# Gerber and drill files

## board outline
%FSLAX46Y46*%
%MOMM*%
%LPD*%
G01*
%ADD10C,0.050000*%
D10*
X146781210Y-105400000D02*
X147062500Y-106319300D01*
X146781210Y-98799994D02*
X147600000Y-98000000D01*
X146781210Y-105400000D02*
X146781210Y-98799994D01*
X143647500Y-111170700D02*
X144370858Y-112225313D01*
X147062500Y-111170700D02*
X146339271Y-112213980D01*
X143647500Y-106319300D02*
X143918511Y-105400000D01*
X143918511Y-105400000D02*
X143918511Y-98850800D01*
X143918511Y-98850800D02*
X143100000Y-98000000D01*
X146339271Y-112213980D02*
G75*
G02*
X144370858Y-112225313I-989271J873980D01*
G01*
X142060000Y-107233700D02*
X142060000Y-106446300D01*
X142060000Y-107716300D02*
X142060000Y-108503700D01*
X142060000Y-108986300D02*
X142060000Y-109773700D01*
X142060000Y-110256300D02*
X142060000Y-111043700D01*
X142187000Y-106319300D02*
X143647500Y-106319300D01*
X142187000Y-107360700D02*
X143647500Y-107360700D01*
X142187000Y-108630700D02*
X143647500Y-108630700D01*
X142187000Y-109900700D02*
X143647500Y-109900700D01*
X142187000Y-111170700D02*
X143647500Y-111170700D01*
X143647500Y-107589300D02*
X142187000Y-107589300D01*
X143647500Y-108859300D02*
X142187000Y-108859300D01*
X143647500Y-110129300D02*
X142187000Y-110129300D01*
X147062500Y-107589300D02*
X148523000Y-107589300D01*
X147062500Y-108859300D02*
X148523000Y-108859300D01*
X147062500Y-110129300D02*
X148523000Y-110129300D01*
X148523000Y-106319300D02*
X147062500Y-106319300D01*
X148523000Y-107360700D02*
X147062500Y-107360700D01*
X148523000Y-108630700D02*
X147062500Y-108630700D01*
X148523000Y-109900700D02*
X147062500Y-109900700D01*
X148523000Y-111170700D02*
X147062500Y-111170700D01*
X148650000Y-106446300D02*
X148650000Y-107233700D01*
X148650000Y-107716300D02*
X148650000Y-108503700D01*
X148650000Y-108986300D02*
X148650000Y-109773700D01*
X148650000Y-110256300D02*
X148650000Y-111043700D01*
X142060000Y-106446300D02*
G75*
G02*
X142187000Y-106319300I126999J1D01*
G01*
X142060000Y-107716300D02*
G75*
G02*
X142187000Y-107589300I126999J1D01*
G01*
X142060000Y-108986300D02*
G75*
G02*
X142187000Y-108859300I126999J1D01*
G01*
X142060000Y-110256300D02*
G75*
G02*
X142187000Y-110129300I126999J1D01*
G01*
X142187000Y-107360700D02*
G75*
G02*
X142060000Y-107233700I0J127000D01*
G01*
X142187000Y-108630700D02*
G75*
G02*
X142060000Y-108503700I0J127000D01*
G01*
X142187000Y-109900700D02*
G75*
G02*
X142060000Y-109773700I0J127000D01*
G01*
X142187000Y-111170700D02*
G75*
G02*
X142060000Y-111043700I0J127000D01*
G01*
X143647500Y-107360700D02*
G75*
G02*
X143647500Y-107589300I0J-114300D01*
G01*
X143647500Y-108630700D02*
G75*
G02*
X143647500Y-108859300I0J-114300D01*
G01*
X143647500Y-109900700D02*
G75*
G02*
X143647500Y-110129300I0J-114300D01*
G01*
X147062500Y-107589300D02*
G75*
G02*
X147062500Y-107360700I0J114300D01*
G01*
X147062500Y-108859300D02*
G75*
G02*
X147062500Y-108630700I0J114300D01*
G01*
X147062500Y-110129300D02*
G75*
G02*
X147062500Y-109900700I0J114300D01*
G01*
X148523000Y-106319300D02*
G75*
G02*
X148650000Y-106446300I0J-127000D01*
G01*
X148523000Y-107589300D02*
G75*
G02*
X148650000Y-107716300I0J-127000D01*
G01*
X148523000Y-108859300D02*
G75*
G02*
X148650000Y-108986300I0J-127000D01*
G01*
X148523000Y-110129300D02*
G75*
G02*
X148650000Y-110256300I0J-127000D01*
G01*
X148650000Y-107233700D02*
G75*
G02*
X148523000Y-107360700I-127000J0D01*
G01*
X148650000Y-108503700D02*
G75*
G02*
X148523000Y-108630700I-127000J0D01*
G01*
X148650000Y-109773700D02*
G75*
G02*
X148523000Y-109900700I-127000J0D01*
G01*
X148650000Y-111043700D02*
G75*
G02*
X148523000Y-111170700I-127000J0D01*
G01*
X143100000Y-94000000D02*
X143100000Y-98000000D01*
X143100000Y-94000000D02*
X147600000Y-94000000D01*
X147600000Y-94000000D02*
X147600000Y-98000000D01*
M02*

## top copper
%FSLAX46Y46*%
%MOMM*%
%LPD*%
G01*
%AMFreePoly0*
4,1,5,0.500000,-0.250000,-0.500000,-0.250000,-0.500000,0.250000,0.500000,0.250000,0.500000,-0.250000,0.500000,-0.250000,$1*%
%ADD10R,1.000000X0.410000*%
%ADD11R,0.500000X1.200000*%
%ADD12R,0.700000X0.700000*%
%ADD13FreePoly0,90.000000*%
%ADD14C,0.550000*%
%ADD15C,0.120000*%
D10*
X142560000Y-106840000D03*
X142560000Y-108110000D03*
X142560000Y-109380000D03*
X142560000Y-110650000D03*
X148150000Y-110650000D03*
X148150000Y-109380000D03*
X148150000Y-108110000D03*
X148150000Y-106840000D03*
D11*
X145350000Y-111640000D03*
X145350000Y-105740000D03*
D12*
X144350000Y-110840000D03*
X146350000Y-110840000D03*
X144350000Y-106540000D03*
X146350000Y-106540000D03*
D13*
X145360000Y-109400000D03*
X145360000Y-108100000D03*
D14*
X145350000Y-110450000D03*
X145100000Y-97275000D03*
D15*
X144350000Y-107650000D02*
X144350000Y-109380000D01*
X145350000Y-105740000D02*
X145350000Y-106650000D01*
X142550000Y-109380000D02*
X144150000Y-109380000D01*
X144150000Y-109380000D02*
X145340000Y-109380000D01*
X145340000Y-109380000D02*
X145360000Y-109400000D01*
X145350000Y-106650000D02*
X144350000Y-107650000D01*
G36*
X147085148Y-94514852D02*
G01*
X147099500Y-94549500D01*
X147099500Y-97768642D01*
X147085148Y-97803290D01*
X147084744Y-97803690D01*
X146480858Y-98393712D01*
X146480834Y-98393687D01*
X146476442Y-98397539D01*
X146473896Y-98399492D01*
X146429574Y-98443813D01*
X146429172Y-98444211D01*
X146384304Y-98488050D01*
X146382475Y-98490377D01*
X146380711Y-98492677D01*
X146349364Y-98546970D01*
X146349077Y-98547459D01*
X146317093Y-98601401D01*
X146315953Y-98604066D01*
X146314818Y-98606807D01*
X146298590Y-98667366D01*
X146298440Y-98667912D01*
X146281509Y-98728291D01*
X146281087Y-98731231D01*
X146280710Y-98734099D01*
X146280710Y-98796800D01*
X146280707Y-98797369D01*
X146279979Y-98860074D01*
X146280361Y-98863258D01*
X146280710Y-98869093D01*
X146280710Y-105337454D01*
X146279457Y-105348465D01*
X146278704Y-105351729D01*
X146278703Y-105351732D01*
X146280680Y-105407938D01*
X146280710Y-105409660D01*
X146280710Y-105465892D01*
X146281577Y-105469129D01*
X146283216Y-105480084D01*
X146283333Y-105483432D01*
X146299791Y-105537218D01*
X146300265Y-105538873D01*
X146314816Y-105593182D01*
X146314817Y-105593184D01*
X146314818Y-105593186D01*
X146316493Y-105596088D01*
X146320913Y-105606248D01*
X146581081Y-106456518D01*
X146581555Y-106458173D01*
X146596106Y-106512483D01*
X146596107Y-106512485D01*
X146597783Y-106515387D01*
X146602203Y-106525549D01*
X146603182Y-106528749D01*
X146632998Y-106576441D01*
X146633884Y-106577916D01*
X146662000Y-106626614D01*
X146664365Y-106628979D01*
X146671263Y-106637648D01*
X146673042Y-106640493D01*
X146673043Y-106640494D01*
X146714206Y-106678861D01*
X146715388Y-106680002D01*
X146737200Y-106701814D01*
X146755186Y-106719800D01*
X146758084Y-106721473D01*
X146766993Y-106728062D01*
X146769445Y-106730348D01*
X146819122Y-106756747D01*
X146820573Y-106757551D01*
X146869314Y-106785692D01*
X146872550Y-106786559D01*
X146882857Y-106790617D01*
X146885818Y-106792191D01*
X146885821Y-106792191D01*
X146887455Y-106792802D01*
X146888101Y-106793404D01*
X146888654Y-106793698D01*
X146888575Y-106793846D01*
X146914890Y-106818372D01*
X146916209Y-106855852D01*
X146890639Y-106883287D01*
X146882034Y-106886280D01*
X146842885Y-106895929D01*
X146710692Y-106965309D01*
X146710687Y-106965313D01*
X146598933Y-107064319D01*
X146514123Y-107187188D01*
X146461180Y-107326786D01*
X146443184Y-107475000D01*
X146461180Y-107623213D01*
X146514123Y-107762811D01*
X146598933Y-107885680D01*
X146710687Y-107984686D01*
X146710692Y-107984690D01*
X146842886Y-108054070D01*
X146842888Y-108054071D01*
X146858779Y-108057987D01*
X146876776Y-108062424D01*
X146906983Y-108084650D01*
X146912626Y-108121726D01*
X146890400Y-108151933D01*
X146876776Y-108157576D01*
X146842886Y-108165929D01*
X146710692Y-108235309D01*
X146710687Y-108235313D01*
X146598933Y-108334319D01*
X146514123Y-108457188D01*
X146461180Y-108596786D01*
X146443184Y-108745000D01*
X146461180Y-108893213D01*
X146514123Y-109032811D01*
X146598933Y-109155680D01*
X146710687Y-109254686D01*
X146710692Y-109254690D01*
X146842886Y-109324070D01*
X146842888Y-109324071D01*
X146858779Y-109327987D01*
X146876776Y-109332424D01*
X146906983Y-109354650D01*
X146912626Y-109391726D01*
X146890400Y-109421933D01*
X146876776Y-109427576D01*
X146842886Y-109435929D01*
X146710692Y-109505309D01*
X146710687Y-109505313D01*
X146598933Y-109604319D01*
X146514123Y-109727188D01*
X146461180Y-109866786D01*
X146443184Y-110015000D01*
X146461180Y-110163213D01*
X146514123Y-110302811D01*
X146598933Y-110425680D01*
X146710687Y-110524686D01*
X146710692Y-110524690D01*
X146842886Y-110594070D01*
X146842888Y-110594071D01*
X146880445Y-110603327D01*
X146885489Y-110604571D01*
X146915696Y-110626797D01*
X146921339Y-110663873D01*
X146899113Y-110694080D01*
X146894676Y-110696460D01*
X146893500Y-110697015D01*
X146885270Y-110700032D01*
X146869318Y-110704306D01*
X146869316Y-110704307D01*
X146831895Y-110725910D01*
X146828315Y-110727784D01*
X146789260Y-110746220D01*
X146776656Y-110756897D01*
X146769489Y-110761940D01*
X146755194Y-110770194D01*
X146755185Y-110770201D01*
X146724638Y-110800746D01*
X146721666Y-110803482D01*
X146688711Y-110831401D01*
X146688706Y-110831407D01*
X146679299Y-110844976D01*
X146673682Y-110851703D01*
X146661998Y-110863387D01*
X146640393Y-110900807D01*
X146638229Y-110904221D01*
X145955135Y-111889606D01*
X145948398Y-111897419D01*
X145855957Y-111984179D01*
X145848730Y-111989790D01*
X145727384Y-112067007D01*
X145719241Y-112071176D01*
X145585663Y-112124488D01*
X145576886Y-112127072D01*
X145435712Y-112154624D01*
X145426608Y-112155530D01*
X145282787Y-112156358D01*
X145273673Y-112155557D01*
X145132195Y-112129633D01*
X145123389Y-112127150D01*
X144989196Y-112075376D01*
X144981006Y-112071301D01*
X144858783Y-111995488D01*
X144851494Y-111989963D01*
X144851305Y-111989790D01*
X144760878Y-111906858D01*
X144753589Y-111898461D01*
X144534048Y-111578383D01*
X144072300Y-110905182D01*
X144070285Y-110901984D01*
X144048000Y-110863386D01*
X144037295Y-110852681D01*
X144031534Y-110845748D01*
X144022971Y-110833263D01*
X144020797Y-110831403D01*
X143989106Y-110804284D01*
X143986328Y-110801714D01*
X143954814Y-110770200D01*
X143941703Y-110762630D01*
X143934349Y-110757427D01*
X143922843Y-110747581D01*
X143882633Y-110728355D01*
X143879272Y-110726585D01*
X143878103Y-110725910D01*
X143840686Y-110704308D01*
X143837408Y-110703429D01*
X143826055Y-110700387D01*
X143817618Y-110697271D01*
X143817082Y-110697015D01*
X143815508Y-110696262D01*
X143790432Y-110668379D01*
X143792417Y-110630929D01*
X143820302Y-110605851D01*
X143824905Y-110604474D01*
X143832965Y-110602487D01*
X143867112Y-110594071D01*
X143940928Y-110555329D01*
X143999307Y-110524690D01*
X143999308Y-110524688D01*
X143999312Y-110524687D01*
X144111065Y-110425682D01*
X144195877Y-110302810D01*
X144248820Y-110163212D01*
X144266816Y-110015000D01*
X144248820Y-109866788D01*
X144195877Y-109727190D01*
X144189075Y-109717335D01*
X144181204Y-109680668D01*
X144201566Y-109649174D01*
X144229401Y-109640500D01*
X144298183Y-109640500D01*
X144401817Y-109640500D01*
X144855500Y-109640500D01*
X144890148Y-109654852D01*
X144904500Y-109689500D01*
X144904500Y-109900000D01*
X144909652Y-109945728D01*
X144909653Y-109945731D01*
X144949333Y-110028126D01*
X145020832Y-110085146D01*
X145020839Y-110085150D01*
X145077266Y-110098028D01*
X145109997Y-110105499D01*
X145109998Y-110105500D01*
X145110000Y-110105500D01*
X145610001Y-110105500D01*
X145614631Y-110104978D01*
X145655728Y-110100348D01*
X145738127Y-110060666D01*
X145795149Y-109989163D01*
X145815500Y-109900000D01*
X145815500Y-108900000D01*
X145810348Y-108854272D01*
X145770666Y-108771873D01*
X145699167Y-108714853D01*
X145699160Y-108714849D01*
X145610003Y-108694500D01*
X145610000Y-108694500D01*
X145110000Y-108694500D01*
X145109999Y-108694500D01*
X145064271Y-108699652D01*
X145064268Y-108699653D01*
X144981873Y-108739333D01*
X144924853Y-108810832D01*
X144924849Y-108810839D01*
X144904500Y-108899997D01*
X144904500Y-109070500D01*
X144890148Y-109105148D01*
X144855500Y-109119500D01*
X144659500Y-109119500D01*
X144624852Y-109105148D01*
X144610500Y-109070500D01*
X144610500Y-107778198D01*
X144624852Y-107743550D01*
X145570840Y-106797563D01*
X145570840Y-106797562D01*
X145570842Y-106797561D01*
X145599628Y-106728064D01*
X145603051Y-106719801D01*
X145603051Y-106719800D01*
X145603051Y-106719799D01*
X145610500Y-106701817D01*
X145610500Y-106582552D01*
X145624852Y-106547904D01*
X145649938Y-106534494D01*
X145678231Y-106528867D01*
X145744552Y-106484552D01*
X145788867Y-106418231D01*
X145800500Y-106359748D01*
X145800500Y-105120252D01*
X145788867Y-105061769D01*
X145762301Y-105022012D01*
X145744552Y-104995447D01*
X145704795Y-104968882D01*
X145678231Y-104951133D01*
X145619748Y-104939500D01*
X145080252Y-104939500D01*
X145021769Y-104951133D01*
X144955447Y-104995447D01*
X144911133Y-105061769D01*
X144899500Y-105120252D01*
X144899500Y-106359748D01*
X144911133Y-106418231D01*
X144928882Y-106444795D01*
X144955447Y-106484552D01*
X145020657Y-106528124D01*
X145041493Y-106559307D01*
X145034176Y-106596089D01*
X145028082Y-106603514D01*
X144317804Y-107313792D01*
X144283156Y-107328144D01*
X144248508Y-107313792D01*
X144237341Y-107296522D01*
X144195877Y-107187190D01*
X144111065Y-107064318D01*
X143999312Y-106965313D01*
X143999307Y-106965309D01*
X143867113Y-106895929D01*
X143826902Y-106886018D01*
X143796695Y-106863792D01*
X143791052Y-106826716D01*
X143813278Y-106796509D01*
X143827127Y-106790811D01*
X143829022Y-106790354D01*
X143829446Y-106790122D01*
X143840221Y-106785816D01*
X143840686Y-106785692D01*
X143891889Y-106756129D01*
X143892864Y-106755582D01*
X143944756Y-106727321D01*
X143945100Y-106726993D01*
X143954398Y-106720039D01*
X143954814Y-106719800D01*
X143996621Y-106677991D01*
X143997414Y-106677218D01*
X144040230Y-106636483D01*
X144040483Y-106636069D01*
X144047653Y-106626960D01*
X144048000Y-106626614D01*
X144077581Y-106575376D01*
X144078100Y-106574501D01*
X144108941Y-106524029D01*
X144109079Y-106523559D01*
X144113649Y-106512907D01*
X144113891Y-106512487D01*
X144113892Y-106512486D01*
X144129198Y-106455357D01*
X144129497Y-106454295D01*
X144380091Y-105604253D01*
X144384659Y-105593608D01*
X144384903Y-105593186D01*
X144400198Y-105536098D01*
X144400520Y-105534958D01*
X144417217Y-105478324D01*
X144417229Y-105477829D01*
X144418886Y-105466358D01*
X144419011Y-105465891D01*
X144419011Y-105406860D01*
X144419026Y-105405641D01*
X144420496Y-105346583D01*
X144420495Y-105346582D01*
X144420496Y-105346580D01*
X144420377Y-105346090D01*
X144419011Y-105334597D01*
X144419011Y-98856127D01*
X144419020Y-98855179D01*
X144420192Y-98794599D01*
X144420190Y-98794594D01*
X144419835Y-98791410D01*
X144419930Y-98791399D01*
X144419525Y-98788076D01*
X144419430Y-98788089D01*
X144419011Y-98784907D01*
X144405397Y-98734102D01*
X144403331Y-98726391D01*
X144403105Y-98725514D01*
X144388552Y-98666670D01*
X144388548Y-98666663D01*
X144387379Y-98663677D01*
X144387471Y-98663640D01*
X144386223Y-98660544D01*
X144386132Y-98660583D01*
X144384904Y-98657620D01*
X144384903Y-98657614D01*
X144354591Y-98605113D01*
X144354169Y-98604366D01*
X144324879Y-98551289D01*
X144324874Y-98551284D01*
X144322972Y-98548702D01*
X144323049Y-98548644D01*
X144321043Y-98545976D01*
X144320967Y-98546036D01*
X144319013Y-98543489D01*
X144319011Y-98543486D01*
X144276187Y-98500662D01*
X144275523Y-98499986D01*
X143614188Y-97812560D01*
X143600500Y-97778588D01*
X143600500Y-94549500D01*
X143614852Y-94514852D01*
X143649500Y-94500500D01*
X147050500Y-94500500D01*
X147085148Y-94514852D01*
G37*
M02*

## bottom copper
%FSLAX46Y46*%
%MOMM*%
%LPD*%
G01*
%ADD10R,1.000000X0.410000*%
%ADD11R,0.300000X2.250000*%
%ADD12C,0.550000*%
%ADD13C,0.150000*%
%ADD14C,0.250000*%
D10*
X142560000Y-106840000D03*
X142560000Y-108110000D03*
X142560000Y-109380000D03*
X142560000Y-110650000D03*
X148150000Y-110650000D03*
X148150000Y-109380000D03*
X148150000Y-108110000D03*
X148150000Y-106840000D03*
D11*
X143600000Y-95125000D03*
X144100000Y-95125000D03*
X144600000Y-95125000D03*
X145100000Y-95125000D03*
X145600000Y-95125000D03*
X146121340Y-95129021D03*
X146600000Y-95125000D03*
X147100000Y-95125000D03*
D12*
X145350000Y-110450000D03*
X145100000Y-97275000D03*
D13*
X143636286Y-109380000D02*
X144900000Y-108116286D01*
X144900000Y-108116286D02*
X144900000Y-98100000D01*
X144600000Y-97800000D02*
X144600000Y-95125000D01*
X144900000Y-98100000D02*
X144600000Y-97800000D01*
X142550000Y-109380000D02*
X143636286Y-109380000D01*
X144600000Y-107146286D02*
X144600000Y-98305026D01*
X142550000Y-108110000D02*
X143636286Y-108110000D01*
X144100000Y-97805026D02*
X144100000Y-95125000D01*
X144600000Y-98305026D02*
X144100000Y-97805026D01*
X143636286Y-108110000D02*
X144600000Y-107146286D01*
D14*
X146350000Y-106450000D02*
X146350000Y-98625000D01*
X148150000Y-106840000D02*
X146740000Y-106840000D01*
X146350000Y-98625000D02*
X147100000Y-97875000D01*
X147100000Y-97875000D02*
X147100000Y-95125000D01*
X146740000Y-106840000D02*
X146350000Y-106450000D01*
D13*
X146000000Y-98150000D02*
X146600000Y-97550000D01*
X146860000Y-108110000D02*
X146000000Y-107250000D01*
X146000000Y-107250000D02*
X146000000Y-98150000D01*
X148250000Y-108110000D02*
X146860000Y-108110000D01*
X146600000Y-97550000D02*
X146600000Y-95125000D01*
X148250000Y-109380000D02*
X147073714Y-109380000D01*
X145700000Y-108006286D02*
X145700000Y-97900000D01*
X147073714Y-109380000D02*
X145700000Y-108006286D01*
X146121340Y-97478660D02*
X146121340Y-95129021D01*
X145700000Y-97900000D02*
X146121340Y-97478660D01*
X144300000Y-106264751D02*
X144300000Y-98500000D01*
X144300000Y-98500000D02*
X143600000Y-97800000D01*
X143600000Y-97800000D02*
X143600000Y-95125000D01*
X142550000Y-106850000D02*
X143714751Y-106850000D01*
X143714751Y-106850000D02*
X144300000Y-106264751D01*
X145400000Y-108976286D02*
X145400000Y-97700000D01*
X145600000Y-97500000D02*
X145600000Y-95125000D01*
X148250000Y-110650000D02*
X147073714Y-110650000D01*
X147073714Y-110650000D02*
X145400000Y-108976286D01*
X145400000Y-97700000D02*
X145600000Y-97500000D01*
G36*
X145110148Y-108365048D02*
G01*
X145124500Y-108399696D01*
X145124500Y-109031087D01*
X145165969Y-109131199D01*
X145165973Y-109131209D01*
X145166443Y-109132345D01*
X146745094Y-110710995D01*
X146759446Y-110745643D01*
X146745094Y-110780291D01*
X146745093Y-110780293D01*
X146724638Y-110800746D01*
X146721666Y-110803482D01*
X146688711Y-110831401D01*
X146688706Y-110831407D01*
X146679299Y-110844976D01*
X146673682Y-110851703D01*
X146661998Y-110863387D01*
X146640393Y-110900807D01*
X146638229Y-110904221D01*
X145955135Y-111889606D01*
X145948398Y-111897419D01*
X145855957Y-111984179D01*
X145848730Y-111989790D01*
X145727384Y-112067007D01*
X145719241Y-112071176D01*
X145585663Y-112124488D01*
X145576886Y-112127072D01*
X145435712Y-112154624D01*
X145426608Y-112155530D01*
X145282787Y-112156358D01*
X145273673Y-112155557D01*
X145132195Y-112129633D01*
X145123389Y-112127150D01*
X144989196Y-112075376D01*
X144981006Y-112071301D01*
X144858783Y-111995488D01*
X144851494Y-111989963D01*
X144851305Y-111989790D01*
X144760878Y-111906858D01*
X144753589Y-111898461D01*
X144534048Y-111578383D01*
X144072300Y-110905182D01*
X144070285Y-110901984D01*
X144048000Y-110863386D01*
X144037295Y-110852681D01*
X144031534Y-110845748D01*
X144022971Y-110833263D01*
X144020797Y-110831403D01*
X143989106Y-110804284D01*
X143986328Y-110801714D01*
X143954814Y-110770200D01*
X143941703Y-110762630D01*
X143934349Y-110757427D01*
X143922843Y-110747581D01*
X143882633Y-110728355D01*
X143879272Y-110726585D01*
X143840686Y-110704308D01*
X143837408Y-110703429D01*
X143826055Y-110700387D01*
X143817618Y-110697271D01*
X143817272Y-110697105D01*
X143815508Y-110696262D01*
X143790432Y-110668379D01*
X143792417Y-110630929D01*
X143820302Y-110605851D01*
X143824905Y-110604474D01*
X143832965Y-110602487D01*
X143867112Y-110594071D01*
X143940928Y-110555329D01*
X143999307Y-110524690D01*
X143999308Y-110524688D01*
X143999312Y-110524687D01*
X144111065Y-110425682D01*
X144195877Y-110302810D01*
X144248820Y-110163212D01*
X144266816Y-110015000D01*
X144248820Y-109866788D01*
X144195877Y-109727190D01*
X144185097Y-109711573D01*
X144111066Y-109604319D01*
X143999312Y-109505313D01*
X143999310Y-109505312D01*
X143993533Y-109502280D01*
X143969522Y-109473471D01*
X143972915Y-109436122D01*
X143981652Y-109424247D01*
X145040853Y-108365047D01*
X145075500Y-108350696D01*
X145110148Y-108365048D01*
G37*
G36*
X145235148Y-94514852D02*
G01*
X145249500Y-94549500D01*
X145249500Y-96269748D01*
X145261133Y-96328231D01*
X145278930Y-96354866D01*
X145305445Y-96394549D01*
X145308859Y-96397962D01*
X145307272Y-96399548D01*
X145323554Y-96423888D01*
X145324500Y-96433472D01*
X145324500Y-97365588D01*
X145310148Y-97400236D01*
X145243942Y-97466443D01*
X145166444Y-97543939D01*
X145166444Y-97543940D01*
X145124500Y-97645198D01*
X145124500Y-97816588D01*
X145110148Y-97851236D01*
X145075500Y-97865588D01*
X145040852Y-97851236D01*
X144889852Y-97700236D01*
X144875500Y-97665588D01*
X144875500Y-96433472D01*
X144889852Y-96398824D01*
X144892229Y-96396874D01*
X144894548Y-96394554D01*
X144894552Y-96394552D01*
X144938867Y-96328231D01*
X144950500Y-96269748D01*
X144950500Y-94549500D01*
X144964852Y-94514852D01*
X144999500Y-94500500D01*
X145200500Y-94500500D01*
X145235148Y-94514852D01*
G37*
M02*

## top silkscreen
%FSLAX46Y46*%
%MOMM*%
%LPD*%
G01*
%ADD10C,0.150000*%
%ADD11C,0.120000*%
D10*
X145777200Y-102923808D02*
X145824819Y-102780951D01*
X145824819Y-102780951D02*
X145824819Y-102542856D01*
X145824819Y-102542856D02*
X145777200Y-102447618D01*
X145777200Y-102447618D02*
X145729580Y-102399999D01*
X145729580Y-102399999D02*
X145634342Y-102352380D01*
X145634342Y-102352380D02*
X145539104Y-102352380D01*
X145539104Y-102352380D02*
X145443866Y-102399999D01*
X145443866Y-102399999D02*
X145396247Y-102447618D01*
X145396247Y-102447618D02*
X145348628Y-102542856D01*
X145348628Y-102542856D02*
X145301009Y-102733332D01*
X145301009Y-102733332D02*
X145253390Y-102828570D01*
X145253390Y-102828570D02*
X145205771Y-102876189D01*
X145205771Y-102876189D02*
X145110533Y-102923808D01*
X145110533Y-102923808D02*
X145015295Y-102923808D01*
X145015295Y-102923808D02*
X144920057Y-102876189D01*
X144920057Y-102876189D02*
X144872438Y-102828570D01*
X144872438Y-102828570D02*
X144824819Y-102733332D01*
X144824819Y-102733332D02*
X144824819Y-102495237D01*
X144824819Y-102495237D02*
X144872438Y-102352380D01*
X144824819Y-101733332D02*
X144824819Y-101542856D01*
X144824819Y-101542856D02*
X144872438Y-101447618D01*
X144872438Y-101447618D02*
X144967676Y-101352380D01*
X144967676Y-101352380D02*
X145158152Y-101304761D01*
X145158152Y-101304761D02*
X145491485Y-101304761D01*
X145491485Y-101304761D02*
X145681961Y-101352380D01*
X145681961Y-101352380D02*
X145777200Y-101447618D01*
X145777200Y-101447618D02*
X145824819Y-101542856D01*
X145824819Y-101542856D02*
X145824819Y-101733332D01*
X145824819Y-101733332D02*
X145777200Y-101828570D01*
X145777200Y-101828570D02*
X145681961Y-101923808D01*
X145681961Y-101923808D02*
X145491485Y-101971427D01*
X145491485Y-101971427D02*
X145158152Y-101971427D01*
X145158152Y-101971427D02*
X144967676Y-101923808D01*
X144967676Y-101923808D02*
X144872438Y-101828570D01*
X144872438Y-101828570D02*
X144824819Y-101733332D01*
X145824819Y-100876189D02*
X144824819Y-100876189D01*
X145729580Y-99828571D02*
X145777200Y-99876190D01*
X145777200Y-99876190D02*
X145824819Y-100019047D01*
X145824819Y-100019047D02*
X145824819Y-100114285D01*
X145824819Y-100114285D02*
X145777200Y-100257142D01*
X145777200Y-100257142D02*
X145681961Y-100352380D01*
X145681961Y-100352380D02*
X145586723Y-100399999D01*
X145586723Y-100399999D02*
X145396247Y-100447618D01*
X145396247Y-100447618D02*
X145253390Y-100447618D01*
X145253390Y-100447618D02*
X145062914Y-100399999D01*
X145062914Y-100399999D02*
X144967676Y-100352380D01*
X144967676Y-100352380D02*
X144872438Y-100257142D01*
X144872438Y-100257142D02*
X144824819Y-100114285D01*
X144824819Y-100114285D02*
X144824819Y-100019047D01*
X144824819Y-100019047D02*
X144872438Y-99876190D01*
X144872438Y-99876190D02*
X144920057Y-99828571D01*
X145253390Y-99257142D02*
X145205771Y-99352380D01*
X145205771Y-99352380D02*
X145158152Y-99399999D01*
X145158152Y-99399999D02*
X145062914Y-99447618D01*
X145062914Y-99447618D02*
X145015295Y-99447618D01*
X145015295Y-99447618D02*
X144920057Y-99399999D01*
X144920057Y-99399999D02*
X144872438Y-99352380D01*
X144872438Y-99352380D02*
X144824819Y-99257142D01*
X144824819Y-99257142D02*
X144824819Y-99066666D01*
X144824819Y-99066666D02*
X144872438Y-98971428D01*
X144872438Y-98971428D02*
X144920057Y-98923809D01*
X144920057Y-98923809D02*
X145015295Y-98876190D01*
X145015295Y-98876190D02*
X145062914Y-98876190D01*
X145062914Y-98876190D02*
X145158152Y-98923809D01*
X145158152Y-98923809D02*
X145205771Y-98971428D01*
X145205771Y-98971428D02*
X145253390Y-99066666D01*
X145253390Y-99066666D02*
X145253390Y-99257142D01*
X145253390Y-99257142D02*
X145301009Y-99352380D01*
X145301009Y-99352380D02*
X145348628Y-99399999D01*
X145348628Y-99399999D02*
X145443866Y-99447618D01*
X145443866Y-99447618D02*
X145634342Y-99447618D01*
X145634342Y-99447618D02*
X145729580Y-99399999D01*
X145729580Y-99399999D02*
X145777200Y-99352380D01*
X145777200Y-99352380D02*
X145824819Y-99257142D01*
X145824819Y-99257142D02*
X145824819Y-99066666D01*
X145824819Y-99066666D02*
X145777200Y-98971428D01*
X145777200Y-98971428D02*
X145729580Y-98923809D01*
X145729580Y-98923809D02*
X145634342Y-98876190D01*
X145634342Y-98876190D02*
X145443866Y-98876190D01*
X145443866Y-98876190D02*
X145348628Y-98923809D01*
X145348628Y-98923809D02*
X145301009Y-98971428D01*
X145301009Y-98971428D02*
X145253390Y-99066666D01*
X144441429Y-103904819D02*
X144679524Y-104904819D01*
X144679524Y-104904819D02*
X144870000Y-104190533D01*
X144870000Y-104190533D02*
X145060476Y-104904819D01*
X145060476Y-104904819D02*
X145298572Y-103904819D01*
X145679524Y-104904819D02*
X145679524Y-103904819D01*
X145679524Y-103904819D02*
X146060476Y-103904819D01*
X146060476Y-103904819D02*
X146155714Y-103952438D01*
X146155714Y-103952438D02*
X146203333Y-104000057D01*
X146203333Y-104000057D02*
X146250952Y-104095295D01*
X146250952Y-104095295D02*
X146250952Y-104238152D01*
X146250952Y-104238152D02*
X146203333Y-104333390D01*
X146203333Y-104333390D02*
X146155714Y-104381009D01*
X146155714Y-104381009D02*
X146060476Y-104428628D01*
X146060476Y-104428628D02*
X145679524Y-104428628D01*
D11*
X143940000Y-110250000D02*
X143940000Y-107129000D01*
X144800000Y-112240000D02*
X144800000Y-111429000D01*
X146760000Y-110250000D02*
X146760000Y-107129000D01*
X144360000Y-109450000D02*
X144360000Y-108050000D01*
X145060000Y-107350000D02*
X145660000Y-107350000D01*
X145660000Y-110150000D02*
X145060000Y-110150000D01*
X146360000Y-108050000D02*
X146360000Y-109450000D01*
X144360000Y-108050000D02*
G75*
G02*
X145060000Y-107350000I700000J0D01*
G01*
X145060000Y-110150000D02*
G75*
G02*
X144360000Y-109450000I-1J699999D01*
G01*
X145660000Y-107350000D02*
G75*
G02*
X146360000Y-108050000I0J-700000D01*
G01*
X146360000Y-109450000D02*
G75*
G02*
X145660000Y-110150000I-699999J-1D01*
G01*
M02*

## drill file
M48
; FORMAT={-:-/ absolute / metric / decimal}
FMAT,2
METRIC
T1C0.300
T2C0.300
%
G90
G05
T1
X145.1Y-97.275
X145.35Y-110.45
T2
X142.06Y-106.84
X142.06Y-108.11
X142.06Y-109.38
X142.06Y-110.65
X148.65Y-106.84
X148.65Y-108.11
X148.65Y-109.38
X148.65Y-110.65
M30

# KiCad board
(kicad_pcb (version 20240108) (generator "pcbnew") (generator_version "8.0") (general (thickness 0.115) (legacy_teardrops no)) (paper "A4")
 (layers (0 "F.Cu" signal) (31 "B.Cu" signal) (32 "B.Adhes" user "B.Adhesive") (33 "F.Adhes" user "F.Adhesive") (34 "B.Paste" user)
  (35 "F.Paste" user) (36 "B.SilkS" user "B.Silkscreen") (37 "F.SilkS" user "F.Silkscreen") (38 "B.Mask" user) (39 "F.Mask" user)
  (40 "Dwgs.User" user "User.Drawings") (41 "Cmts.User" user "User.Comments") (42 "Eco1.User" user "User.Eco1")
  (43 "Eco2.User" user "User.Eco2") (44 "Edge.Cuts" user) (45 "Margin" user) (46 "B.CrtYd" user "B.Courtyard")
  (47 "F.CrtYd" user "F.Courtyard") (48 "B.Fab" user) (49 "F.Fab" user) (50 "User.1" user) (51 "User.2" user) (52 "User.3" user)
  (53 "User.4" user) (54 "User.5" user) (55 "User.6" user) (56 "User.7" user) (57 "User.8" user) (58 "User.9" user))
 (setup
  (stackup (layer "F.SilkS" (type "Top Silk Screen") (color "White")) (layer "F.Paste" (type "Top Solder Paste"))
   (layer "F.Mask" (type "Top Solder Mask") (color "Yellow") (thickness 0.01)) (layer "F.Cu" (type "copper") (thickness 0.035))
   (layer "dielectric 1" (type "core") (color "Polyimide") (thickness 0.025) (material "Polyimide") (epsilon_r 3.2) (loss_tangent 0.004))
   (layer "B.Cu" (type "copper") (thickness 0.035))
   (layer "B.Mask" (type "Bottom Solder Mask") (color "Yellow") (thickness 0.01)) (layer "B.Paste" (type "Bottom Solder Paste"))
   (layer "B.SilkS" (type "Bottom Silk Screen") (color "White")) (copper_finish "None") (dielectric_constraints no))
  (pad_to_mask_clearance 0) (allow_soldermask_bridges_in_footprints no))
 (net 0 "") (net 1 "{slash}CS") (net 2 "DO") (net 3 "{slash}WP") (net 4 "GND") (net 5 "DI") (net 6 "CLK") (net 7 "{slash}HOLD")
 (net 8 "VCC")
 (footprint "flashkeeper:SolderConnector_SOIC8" (layer "F.Cu") (at 142.06 106.84)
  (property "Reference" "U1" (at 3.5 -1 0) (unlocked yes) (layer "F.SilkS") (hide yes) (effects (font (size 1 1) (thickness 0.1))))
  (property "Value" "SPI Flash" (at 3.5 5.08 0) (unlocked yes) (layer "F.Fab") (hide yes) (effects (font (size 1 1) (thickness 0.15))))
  (fp_line (start 0 0.3937) (end 0 -0.3937) (stroke (width 0.05) (type default)) (layer "Edge.Cuts"))
  (fp_line (start 0 0.8763) (end 0 1.6637) (stroke (width 0.05) (type default)) (layer "Edge.Cuts"))
  (fp_line (start 0 2.1463) (end 0 2.9337) (stroke (width 0.05) (type default)) (layer "Edge.Cuts"))
  (fp_line (start 0 3.4163) (end 0 4.2037) (stroke (width 0.05) (type default)) (layer "Edge.Cuts"))
  (fp_line (start 0.127 -0.5207) (end 1.5875 -0.5207) (stroke (width 0.05) (type default)) (layer "Edge.Cuts"))
  (fp_line (start 0.127 0.5207) (end 1.5875 0.5207) (stroke (width 0.05) (type default)) (layer "Edge.Cuts"))
  (fp_line (start 0.127 1.7907) (end 1.5875 1.7907) (stroke (width 0.05) (type default)) (layer "Edge.Cuts"))
  (fp_line (start 0.127 3.0607) (end 1.5875 3.0607) (stroke (width 0.05) (type default)) (layer "Edge.Cuts"))
  (fp_line (start 0.127 4.3307) (end 1.5875 4.3307) (stroke (width 0.05) (type default)) (layer "Edge.Cuts"))
  (fp_line (start 1.5875 0.7493) (end 0.127 0.7493) (stroke (width 0.05) (type default)) (layer "Edge.Cuts"))
  (fp_line (start 1.5875 2.0193) (end 0.127 2.0193) (stroke (width 0.05) (type default)) (layer "Edge.Cuts"))
  (fp_line (start 1.5875 3.2893) (end 0.127 3.2893) (stroke (width 0.05) (type default)) (layer "Edge.Cuts"))
  (fp_line (start 5.0025 0.7493) (end 6.463 0.7493) (stroke (width 0.05) (type default)) (layer "Edge.Cuts"))
  (fp_line (start 5.0025 2.0193) (end 6.463 2.0193) (stroke (width 0.05) (type default)) (layer "Edge.Cuts"))
  (fp_line (start 5.0025 3.2893) (end 6.463 3.2893) (stroke (width 0.05) (type default)) (layer "Edge.Cuts"))
  (fp_line (start 6.463 -0.5207) (end 5.0025 -0.5207) (stroke (width 0.05) (type default)) (layer "Edge.Cuts"))
  (fp_line (start 6.463 0.5207) (end 5.0025 0.5207) (stroke (width 0.05) (type default)) (layer "Edge.Cuts"))
  (fp_line (start 6.463 1.7907) (end 5.0025 1.7907) (stroke (width 0.05) (type default)) (layer "Edge.Cuts"))
  (fp_line (start 6.463 3.0607) (end 5.0025 3.0607) (stroke (width 0.05) (type default)) (layer "Edge.Cuts"))
  (fp_line (start 6.463 4.3307) (end 5.0025 4.3307) (stroke (width 0.05) (type default)) (layer "Edge.Cuts"))
  (fp_line (start 6.59 -0.3937) (end 6.59 0.3937) (stroke (width 0.05) (type default)) (layer "Edge.Cuts"))
  (fp_line (start 6.59 0.8763) (end 6.59 1.6637) (stroke (width 0.05) (type default)) (layer "Edge.Cuts"))
  (fp_line (start 6.59 2.1463) (end 6.59 2.9337) (stroke (width 0.05) (type default)) (layer "Edge.Cuts"))
  (fp_line (start 6.59 3.4163) (end 6.59 4.2037) (stroke (width 0.05) (type default)) (layer "Edge.Cuts"))
  (fp_arc (start 0 -0.3937) (mid 0.037197 -0.483503) (end 0.127 -0.5207) (stroke (width 0.05) (type default)) (layer "Edge.Cuts"))
  (fp_arc (start 0 0.8763) (mid 0.037197 0.786497) (end 0.127 0.7493) (stroke (width 0.05) (type default)) (layer "Edge.Cuts"))
  (fp_arc (start 0 2.1463) (mid 0.037197 2.056497) (end 0.127 2.0193) (stroke (width 0.05) (type default)) (layer "Edge.Cuts"))
  (fp_arc (start 0 3.4163) (mid 0.037197 3.326497) (end 0.127 3.2893) (stroke (width 0.05) (type default)) (layer "Edge.Cuts"))
  (fp_arc (start 0.127 0.5207) (mid 0.037197 0.483503) (end 0 0.3937) (stroke (width 0.05) (type default)) (layer "Edge.Cuts"))
  (fp_arc (start 0.127 1.7907) (mid 0.037197 1.753503) (end 0 1.6637) (stroke (width 0.05) (type default)) (layer "Edge.Cuts"))
  (fp_arc (start 0.127 3.0607) (mid 0.037197 3.023503) (end 0 2.9337) (stroke (width 0.05) (type default)) (layer "Edge.Cuts"))
  (fp_arc (start 0.127 4.3307) (mid 0.037197 4.293503) (end 0 4.2037) (stroke (width 0.05) (type default)) (layer "Edge.Cuts"))
  (fp_arc (start 1.5875 0.5207) (mid 1.7018 0.635) (end 1.5875 0.7493) (stroke (width 0.05) (type default)) (layer "Edge.Cuts"))
  (fp_arc (start 1.5875 1.7907) (mid 1.7018 1.905) (end 1.5875 2.0193) (stroke (width 0.05) (type default)) (layer "Edge.Cuts"))
  (fp_arc (start 1.5875 3.0607) (mid 1.7018 3.175) (end 1.5875 3.2893) (stroke (width 0.05) (type default)) (layer "Edge.Cuts"))
  (fp_arc (start 5.0025 0.7493) (mid 4.8882 0.635) (end 5.0025 0.5207) (stroke (width 0.05) (type default)) (layer "Edge.Cuts"))
  (fp_arc (start 5.0025 2.0193) (mid 4.8882 1.905) (end 5.0025 1.7907) (stroke (width 0.05) (type default)) (layer "Edge.Cuts"))
  (fp_arc (start 5.0025 3.2893) (mid 4.8882 3.175) (end 5.0025 3.0607) (stroke (width 0.05) (type default)) (layer "Edge.Cuts"))
  (fp_arc (start 6.463 -0.5207) (mid 6.552803 -0.483503) (end 6.59 -0.3937) (stroke (width 0.05) (type default)) (layer "Edge.Cuts"))
  (fp_arc (start 6.463 0.7493) (mid 6.552803 0.786497) (end 6.59 0.8763) (stroke (width 0.05) (type default)) (layer "Edge.Cuts"))
  (fp_arc (start 6.463 2.0193) (mid 6.552803 2.056497) (end 6.59 2.1463) (stroke (width 0.05) (type default)) (layer "Edge.Cuts"))
  (fp_arc (start 6.463 3.2893) (mid 6.552803 3.326497) (end 6.59 3.4163) (stroke (width 0.05) (type default)) (layer "Edge.Cuts"))
  (fp_arc (start 6.59 0.3937) (mid 6.552803 0.483503) (end 6.463 0.5207) (stroke (width 0.05) (type default)) (layer "Edge.Cuts"))
  (fp_arc (start 6.59 1.6637) (mid 6.552803 1.753503) (end 6.463 1.7907) (stroke (width 0.05) (type default)) (layer "Edge.Cuts"))
  (fp_arc (start 6.59 2.9337) (mid 6.552803 3.023503) (end 6.463 3.0607) (stroke (width 0.05) (type default)) (layer "Edge.Cuts"))
  (fp_arc (start 6.59 4.2037) (mid 6.552803 4.293503) (end 6.463 4.3307) (stroke (width 0.05) (type default)) (layer "Edge.Cuts"))
  (pad "1" thru_hole rect (at 0 0) (size 1 0.41) (drill 0.3 (offset 0.5 0)) (layers "*.Cu" "*.Mask") (remove_unused_layers no)
   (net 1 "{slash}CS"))
  (pad "2" thru_hole rect (at 0 1.27) (size 1 0.41) (drill 0.3 (offset 0.5 0)) (layers "*.Cu" "*.Mask") (remove_unused_layers no)
   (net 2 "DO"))
  (pad "3" thru_hole rect (at 0 2.54) (size 1 0.41) (drill 0.3 (offset 0.5 0)) (layers "*.Cu" "*.Mask") (remove_unused_layers no)
   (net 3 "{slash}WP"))
  (pad "4" thru_hole rect (at 0 3.81) (size 1 0.41) (drill 0.3 (offset 0.5 0)) (layers "*.Cu" "*.Mask") (remove_unused_layers no)
   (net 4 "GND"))
  (pad "5" thru_hole rect (at 6.59 3.81 180) (size 1 0.41) (drill 0.3 (offset 0.5 0)) (layers "*.Cu" "*.Mask") (remove_unused_layers no)
   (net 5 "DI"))
  (pad "6" thru_hole rect (at 6.59 2.54 180) (size 1 0.41) (drill 0.3 (offset 0.5 0)) (layers "*.Cu" "*.Mask") (remove_unused_layers no)
   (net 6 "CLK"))
  (pad "7" thru_hole rect (at 6.59 1.27 180) (size 1 0.41) (drill 0.3 (offset 0.5 0)) (layers "*.Cu" "*.Mask") (remove_unused_layers no)
   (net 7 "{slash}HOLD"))
  (pad "8" thru_hole rect (at 6.59 0 180) (size 1 0.41) (drill 0.3 (offset 0.5 0)) (layers "*.Cu" "*.Mask") (remove_unused_layers no)
   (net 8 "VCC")))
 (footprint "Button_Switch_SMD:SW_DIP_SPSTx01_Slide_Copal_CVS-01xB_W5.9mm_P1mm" (layer "F.Cu") (at 145.35 108.69 90)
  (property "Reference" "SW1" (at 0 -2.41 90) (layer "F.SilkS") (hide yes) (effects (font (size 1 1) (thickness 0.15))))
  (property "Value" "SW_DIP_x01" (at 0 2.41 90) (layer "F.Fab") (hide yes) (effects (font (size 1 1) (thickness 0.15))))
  (fp_line (start -1.56 -1.41) (end 1.561 -1.41) (stroke (width 0.12) (type solid)) (layer "F.SilkS"))
  (fp_line (start -3.55 -0.55) (end -2.739 -0.55) (stroke (width 0.12) (type solid)) (layer "F.SilkS"))
  (fp_line (start -1.56 1.41) (end 1.561 1.41) (stroke (width 0.12) (type solid)) (layer "F.SilkS"))
  (pad "1" smd rect (at -2.95 0 90) (size 1.2 0.5) (layers "F.Cu" "F.Paste" "F.Mask") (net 4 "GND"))
  (pad "2" smd rect (at 2.95 0 90) (size 1.2 0.5) (layers "F.Cu" "F.Paste" "F.Mask") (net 3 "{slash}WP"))
  (pad "3" smd rect (at -2.15 -1 90) (size 0.7 0.7) (layers "F.Cu" "F.Paste" "F.Mask") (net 4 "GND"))
  (pad "3" smd rect (at -2.15 1 90) (size 0.7 0.7) (layers "F.Cu" "F.Paste" "F.Mask") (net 4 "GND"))
  (pad "3" smd rect (at 2.15 -1 90) (size 0.7 0.7) (layers "F.Cu" "F.Paste" "F.Mask") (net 4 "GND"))
  (pad "3" smd rect (at 2.15 1 90) (size 0.7 0.7) (layers "F.Cu" "F.Paste" "F.Mask") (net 4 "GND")))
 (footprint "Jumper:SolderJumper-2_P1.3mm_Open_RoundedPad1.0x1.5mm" (layer "F.Cu") (at 145.36 108.75 90)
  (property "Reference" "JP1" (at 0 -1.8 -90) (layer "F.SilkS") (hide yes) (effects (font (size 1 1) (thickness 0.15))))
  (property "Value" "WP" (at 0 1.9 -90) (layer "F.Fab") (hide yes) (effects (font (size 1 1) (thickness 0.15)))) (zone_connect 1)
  (fp_line (start -0.7 -1) (end 0.7 -1) (stroke (width 0.12) (type solid)) (layer "F.SilkS"))
  (fp_line (start 1.4 -0.3) (end 1.4 0.3) (stroke (width 0.12) (type solid)) (layer "F.SilkS"))
  (fp_line (start -1.4 0.3) (end -1.4 -0.3) (stroke (width 0.12) (type solid)) (layer "F.SilkS"))
  (fp_line (start 0.7 1) (end -0.7 1) (stroke (width 0.12) (type solid)) (layer "F.SilkS"))
  (fp_arc (start 0.7 -1) (mid 1.194975 -0.794975) (end 1.4 -0.3) (stroke (width 0.12) (type solid)) (layer "F.SilkS"))
  (fp_arc (start -1.4 -0.3) (mid -1.194975 -0.794975) (end -0.7 -1) (stroke (width 0.12) (type solid)) (layer "F.SilkS"))
  (fp_arc (start 1.4 0.3) (mid 1.194975 0.794975) (end 0.7 1) (stroke (width 0.12) (type solid)) (layer "F.SilkS"))
  (fp_arc (start -0.7 1) (mid -1.194975 0.794975) (end -1.4 0.3) (stroke (width 0.12) (type solid)) (layer "F.SilkS"))
  (pad "1" smd custom (at -0.65 0 90) (size 1 0.5) (layers "F.Cu" "F.Mask") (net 3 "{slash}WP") (zone_connect 2) (thermal_bridge_angle 45)
   (options (clearance outline) (anchor rect)) (primitives))
  (pad "2" smd custom (at 0.65 0 90) (size 1 0.5) (layers "F.Cu" "F.Mask") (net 4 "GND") (zone_connect 2) (thermal_bridge_angle 45)
   (options (clearance outline) (anchor rect)) (primitives)))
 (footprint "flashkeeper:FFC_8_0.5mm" (layer "F.Cu") (at 145.35 94)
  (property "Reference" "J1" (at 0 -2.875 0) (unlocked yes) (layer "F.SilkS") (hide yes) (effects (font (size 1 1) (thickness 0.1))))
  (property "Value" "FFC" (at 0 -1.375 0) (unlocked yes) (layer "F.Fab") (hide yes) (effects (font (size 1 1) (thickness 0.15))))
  (fp_line (start -2.25 0) (end -2.25 4) (stroke (width 0.05) (type default)) (layer "Edge.Cuts"))
  (fp_line (start -2.25 0) (end 2.25 0) (stroke (width 0.05) (type default)) (layer "Edge.Cuts"))
  (fp_line (start 2.25 0) (end 2.25 4) (stroke (width 0.05) (type default)) (layer "Edge.Cuts"))
  (pad "1" smd rect (at -1.75 1.125) (size 0.3 2.25) (layers "B.Cu" "B.Mask") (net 1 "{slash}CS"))
  (pad "2" smd rect (at -1.25 1.125) (size 0.3 2.25) (layers "B.Cu" "B.Mask") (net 2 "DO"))
  (pad "3" smd rect (at -0.75 1.125) (size 0.3 2.25) (layers "B.Cu" "B.Mask") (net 3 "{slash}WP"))
  (pad "4" smd rect (at -0.25 1.125) (size 0.3 2.25) (layers "B.Cu" "B.Mask") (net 4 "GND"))
  (pad "5" smd rect (at 0.25 1.125) (size 0.3 2.25) (layers "B.Cu" "B.Mask") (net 5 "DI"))
  (pad "6" smd rect (at 0.77134 1.129021) (size 0.3 2.25) (layers "B.Cu" "B.Mask") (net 6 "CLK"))
  (pad "7" smd rect (at 1.25 1.125) (size 0.3 2.25) (layers "B.Cu" "B.Mask") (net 7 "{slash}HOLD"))
  (pad "8" smd rect (at 1.75 1.125) (size 0.3 2.25) (layers "B.Cu" "B.Mask") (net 8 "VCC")))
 (gr_line (start 146.78121 105.4) (end 147.0625 106.3193) (stroke (width 0.05) (type default)) (layer "Edge.Cuts"))
 (gr_line (start 146.78121 98.799994) (end 147.6 98) (stroke (width 0.05) (type default)) (layer "Edge.Cuts"))
 (gr_line (start 146.78121 105.4) (end 146.78121 98.799994) (stroke (width 0.05) (type default)) (layer "Edge.Cuts"))
 (gr_line (start 143.6475 111.1707) (end 144.370858 112.225313) (stroke (width 0.05) (type default)) (layer "Edge.Cuts"))
 (gr_line (start 147.0625 111.1707) (end 146.339271 112.21398) (stroke (width 0.05) (type default)) (layer "Edge.Cuts"))
 (gr_line (start 143.6475 106.3193) (end 143.918511 105.4) (stroke (width 0.05) (type default)) (layer "Edge.Cuts"))
 (gr_line (start 143.918511 105.4) (end 143.918511 98.8508) (stroke (width 0.05) (type default)) (layer "Edge.Cuts"))
 (gr_line (start 143.918511 98.8508) (end 143.1 98) (stroke (width 0.05) (type default)) (layer "Edge.Cuts"))
 (gr_arc (start 146.339271 112.21398) (mid 145.3576 112.660015) (end 144.370858 112.225313) (stroke (width 0.05) (type default))
  (layer "Edge.Cuts"))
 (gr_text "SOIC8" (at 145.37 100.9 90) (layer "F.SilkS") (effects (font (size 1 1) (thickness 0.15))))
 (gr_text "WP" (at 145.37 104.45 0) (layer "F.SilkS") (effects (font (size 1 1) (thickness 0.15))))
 (segment (start 144.35 107.65) (end 144.35 109.38) (width 0.12) (layer "F.Cu") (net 3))
 (segment (start 145.35 105.74) (end 145.35 106.65) (width 0.12) (layer "F.Cu") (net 3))
 (segment (start 142.55 109.38) (end 144.15 109.38) (width 0.12) (layer "F.Cu") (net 3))
 (segment (start 144.15 109.38) (end 145.34 109.38) (width 0.12) (layer "F.Cu") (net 3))
 (segment (start 145.34 109.38) (end 145.36 109.4) (width 0.12) (layer "F.Cu") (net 3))
 (segment (start 145.35 106.65) (end 144.35 107.65) (width 0.12) (layer "F.Cu") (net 3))
 (segment (start 143.636286 109.38) (end 144.9 108.116286) (width 0.15) (layer "B.Cu") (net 3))
 (segment (start 144.9 108.116286) (end 144.9 98.1) (width 0.15) (layer "B.Cu") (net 3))
 (segment (start 144.6 97.8) (end 144.6 95.125) (width 0.15) (layer "B.Cu") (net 3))
 (segment (start 144.9 98.1) (end 144.6 97.8) (width 0.15) (layer "B.Cu") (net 3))
 (segment (start 142.55 109.38) (end 143.636286 109.38) (width 0.15) (layer "B.Cu") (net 3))
 (via (at 145.35 110.45) (size 0.55) (drill 0.3) (layers "F.Cu" "B.Cu") (free yes) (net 4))
 (via (at 145.1 97.275) (size 0.55) (drill 0.3) (layers "F.Cu" "B.Cu") (free yes) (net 4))
 (segment (start 144.6 107.146286) (end 144.6 98.305026) (width 0.15) (layer "B.Cu") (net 2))
 (segment (start 142.55 108.11) (end 143.636286 108.11) (width 0.15) (layer "B.Cu") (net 2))
 (segment (start 144.1 97.805026) (end 144.1 95.125) (width 0.15) (layer "B.Cu") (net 2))
 (segment (start 144.6 98.305026) (end 144.1 97.805026) (width 0.15) (layer "B.Cu") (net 2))
 (segment (start 143.636286 108.11) (end 144.6 107.146286) (width 0.15) (layer "B.Cu") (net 2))
 (segment (start 146.35 106.45) (end 146.35 98.625) (width 0.25) (layer "B.Cu") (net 8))
 (segment (start 148.15 106.84) (end 146.74 106.84) (width 0.25) (layer "B.Cu") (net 8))
 (segment (start 146.35 98.625) (end 147.1 97.875) (width 0.25) (layer "B.Cu") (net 8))
 (segment (start 147.1 97.875) (end 147.1 95.125) (width 0.25) (layer "B.Cu") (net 8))
 (segment (start 146.74 106.84) (end 146.35 106.45) (width 0.25) (layer "B.Cu") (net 8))
 (segment (start 146 98.15) (end 146.6 97.55) (width 0.15) (layer "B.Cu") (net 7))
 (segment (start 146.86 108.11) (end 146 107.25) (width 0.15) (layer "B.Cu") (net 7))
 (segment (start 146 107.25) (end 146 98.15) (width 0.15) (layer "B.Cu") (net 7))
 (segment (start 148.25 108.11) (end 146.86 108.11) (width 0.15) (layer "B.Cu") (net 7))
 (segment (start 146.6 97.55) (end 146.6 95.125) (width 0.15) (layer "B.Cu") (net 7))
 (segment (start 148.25 109.38) (end 147.073714 109.38) (width 0.15) (layer "B.Cu") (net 6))
 (segment (start 145.7 108.006286) (end 145.7 97.9) (width 0.15) (layer "B.Cu") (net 6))
 (segment (start 147.073714 109.38) (end 145.7 108.006286) (width 0.15) (layer "B.Cu") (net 6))
 (segment (start 146.12134 97.47866) (end 146.12134 95.129021) (width 0.15) (layer "B.Cu") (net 6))
 (segment (start 145.7 97.9) (end 146.12134 97.47866) (width 0.15) (layer "B.Cu") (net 6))
 (segment (start 144.3 106.264751) (end 144.3 98.5) (width 0.15) (layer "B.Cu") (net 1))
 (segment (start 144.3 98.5) (end 143.6 97.8) (width 0.15) (layer "B.Cu") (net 1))
 (segment (start 143.6 97.8) (end 143.6 95.125) (width 0.15) (layer "B.Cu") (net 1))
 (segment (start 142.55 106.85) (end 143.714751 106.85) (width 0.15) (layer "B.Cu") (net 1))
 (segment (start 143.714751 106.85) (end 144.3 106.264751) (width 0.15) (layer "B.Cu") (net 1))
 (segment (start 145.4 108.976286) (end 145.4 97.7) (width 0.15) (layer "B.Cu") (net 5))
 (segment (start 145.6 97.5) (end 145.6 95.125) (width 0.15) (layer "B.Cu") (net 5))
 (segment (start 148.25 110.65) (end 147.073714 110.65) (width 0.15) (layer "B.Cu") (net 5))
 (segment (start 147.073714 110.65) (end 145.4 108.976286) (width 0.15) (layer "B.Cu") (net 5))
 (segment (start 145.4 97.7) (end 145.6 97.5) (width 0.15) (layer "B.Cu") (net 5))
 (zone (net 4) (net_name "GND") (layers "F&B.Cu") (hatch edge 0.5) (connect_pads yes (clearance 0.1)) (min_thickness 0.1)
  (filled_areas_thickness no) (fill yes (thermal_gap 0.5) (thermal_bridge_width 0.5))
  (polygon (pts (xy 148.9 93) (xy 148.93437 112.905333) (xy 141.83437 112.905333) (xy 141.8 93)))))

